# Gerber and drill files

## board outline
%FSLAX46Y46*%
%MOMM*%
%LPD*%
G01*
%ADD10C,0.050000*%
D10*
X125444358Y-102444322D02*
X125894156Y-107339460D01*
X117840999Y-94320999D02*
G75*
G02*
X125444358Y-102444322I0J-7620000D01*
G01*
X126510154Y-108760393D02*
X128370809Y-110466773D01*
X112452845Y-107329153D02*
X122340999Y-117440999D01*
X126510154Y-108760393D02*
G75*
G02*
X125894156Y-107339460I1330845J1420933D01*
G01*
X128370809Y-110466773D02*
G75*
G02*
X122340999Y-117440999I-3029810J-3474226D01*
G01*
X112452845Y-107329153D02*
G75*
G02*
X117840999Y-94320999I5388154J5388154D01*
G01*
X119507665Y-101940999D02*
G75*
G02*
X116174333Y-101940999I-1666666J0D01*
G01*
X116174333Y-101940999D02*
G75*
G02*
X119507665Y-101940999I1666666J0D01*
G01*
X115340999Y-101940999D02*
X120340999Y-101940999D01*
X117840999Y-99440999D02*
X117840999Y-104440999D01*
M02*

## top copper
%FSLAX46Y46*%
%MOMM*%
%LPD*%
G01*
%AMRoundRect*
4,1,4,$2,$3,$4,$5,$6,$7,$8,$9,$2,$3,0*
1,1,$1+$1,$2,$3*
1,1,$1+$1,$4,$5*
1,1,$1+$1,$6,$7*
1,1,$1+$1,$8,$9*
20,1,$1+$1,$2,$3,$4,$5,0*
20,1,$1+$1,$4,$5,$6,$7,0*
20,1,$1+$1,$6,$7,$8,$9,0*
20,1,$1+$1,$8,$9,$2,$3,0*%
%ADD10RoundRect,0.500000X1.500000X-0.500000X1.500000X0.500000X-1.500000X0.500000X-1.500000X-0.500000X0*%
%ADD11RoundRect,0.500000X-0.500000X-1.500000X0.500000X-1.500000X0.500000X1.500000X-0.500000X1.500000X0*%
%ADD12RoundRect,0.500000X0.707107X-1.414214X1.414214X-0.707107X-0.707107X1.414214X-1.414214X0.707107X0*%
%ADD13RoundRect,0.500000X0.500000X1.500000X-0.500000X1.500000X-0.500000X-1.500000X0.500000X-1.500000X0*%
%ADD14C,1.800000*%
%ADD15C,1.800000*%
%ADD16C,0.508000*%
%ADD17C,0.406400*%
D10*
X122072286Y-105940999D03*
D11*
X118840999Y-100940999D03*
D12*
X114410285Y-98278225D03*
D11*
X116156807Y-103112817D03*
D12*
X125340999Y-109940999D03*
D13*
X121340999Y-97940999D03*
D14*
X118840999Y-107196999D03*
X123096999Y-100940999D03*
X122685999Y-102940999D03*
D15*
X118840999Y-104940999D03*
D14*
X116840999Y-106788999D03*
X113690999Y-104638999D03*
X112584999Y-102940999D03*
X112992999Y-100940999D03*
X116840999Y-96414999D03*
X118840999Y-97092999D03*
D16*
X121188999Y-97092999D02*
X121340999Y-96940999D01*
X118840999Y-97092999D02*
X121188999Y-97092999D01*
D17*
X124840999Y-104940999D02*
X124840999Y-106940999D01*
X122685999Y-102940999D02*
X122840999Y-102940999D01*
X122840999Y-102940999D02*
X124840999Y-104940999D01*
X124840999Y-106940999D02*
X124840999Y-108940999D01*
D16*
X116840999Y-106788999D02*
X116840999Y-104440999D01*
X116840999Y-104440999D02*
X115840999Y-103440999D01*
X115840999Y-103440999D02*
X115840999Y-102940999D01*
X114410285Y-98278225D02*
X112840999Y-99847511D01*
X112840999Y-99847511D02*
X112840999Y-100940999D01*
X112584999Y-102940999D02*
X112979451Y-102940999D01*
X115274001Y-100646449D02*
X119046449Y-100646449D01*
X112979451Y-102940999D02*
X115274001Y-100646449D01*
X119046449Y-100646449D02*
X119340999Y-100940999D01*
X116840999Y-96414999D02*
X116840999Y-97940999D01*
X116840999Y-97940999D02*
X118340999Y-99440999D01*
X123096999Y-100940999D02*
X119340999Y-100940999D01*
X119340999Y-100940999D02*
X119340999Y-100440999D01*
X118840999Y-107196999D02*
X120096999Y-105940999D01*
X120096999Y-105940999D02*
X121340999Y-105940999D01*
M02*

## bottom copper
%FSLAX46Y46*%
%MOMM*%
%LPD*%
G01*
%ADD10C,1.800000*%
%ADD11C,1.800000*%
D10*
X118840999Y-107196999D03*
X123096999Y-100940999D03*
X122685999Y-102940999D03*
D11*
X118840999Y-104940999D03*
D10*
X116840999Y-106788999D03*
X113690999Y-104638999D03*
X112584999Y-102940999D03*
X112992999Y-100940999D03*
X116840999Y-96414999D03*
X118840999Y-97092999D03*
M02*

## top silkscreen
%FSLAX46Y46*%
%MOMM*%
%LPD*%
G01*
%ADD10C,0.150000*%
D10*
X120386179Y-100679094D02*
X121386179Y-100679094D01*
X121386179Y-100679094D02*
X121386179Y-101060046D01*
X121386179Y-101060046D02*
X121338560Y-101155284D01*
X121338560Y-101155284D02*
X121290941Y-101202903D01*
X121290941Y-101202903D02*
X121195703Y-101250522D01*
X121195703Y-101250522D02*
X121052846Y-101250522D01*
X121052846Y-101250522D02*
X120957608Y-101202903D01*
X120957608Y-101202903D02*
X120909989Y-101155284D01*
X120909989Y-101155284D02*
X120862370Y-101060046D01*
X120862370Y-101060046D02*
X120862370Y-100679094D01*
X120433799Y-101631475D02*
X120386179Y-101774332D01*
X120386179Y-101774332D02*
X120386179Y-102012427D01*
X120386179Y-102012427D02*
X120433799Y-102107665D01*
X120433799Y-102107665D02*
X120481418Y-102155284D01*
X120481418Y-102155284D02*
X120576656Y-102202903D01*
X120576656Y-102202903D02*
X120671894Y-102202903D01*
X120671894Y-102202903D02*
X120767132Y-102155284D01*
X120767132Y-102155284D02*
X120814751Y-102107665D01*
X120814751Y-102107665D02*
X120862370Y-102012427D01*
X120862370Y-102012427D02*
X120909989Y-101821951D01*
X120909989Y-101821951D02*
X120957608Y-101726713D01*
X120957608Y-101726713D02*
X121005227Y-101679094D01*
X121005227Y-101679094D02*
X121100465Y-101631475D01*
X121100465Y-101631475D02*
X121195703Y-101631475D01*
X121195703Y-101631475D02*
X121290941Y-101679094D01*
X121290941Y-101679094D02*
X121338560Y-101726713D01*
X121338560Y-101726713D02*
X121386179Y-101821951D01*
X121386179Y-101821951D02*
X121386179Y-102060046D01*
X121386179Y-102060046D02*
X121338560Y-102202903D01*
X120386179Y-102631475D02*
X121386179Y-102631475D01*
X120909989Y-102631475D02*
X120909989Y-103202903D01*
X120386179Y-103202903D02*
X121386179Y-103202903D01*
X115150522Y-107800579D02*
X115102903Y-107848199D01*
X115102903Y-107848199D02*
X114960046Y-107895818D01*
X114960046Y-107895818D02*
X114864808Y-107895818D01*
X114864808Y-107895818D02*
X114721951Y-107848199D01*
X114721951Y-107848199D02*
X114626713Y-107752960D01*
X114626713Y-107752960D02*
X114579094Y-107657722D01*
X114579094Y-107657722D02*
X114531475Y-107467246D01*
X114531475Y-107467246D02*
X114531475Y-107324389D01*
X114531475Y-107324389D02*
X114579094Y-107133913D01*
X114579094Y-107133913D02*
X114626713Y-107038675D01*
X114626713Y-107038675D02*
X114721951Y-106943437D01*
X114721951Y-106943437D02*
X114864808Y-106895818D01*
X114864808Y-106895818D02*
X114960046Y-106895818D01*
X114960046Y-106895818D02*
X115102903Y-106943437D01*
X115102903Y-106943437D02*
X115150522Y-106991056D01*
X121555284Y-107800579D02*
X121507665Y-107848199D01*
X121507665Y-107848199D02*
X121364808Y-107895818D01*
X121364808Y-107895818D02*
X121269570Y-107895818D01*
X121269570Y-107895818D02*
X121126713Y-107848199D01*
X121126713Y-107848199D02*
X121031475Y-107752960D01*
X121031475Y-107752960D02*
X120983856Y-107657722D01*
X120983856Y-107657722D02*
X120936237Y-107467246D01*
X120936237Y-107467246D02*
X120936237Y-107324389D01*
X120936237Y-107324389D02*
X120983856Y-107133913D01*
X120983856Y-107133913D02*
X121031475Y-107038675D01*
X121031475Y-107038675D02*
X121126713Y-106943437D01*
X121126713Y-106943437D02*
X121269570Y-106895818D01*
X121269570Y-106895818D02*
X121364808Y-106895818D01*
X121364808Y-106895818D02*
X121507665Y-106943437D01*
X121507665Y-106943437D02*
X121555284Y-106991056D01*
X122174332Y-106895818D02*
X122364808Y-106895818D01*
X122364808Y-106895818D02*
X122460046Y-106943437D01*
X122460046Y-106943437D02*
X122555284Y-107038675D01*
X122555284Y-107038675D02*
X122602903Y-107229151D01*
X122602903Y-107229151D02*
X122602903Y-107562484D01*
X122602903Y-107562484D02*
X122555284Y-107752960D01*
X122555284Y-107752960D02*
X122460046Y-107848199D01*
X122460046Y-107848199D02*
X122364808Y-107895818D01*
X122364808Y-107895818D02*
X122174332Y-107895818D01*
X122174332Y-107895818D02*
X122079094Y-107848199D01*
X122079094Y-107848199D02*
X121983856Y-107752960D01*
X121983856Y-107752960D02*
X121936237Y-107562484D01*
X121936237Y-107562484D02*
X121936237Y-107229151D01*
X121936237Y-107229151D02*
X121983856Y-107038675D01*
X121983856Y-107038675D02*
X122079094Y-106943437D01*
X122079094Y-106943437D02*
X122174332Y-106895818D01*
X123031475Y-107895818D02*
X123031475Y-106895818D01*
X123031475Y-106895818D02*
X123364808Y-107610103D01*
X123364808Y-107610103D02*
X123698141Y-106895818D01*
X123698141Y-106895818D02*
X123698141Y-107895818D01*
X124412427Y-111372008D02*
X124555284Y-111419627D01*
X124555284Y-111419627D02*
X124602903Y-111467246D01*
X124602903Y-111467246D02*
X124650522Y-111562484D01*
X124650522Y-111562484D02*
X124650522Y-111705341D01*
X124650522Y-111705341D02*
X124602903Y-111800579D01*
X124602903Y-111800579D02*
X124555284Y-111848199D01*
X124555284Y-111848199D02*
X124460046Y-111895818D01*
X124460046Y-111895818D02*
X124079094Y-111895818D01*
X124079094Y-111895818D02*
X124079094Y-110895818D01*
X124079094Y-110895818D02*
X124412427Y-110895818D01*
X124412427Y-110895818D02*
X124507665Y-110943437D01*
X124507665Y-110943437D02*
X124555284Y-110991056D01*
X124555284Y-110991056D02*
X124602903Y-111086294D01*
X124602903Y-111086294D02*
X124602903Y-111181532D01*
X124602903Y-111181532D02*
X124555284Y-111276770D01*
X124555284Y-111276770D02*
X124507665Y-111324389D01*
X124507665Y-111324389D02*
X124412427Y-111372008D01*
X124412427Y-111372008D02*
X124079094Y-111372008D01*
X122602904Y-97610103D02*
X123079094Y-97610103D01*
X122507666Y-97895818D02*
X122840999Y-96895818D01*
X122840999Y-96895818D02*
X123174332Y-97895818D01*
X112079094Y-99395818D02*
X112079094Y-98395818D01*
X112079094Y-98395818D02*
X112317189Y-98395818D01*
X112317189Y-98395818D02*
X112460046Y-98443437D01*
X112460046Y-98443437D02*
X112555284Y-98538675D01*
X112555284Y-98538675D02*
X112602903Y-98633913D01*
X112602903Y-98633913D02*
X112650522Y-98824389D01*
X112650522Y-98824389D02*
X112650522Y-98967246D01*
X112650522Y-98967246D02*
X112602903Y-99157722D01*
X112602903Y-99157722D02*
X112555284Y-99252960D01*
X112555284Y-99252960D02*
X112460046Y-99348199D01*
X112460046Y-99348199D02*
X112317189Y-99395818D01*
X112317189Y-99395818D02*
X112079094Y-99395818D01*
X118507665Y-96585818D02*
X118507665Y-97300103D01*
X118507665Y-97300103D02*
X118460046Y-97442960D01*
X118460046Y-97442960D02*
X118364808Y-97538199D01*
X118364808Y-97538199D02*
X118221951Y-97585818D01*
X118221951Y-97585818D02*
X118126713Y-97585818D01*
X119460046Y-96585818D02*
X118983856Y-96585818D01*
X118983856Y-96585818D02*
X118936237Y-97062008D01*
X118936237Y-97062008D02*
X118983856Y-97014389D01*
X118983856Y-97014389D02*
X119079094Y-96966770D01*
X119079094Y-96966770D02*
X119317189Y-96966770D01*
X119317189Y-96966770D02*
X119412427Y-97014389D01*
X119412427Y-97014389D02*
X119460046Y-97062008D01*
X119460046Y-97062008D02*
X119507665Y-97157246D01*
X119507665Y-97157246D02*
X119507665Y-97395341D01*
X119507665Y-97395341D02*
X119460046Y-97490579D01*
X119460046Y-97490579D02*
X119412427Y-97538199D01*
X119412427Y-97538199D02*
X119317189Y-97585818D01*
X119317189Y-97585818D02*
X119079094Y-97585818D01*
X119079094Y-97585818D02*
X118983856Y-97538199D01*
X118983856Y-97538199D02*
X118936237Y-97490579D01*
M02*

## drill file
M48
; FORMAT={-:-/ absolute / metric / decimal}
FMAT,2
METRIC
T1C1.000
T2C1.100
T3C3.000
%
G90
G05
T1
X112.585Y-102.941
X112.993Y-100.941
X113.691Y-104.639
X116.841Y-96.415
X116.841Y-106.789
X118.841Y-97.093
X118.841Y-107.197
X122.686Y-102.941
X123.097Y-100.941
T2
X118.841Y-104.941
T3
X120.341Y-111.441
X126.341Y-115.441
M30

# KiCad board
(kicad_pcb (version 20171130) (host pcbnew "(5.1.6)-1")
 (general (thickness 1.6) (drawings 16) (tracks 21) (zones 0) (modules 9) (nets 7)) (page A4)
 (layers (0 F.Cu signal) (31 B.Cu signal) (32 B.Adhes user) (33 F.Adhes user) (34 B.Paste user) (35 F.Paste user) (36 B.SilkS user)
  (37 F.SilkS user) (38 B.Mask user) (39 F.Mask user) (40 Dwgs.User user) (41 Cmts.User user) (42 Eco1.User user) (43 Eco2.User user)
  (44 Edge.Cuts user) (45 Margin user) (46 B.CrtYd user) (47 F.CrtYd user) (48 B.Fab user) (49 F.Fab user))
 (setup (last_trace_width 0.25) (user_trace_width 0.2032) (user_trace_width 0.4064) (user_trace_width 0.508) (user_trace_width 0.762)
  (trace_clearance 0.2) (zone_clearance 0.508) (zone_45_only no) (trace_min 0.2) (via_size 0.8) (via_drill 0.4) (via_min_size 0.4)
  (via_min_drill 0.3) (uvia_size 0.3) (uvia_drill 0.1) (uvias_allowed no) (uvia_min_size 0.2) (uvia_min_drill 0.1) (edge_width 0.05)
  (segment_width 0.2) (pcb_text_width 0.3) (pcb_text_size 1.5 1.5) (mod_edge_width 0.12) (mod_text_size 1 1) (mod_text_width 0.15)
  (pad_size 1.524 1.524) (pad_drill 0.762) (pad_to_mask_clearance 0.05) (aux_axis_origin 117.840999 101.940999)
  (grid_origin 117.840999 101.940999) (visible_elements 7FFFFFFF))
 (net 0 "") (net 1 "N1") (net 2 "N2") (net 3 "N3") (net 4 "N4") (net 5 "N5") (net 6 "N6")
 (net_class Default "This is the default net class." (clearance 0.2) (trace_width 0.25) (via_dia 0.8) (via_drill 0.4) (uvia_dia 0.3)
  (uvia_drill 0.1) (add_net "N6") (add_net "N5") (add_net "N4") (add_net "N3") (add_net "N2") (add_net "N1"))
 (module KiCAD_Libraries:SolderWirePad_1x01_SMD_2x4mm (layer F.Cu) (at 122.072286 105.940999 90)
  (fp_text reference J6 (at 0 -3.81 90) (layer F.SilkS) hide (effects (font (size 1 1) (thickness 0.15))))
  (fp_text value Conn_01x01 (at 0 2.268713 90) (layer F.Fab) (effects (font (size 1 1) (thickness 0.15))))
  (pad 1 smd roundrect (at 0 0 90) (size 2 4) (layers F.Cu F.Paste F.Mask) (roundrect_rratio 0.25) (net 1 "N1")))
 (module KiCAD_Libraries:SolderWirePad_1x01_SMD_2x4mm (layer F.Cu) (at 118.840999 100.940999)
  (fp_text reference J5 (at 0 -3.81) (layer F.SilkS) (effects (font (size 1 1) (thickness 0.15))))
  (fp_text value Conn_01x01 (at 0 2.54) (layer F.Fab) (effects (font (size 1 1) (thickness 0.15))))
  (pad 1 smd roundrect (at 0 0) (size 2 4) (layers F.Cu F.Paste F.Mask) (roundrect_rratio 0.25) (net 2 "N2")))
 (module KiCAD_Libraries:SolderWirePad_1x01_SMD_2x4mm (layer F.Cu) (at 114.410285 98.278225 45)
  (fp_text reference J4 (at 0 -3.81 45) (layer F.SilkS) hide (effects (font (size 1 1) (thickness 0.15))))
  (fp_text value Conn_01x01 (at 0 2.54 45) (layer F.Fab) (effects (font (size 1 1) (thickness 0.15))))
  (pad 1 smd roundrect (at 0 0 45) (size 2 4) (layers F.Cu F.Paste F.Mask) (roundrect_rratio 0.25) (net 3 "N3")))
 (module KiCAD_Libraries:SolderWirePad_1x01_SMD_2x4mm (layer F.Cu) (at 116.156807 103.112817)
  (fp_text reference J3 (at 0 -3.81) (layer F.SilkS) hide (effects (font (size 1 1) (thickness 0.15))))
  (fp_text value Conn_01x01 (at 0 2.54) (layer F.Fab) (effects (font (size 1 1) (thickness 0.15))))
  (pad 1 smd roundrect (at 0 0) (size 2 4) (layers F.Cu F.Paste F.Mask) (roundrect_rratio 0.25) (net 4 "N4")))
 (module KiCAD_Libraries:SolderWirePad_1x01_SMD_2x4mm (layer F.Cu) (at 125.340999 109.940999 45)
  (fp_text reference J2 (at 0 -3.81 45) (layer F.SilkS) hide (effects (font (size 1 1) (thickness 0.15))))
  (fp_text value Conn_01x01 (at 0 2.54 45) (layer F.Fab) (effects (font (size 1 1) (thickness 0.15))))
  (pad 1 smd roundrect (at 0 0 45) (size 2 4) (layers F.Cu F.Paste F.Mask) (roundrect_rratio 0.25) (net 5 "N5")))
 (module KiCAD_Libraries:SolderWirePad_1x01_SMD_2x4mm (layer F.Cu) (at 121.340999 97.940999 180)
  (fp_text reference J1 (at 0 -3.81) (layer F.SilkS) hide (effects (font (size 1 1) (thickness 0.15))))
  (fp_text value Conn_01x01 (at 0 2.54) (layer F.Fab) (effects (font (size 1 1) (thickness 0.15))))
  (pad 1 smd roundrect (at 0 0 180) (size 2 4) (layers F.Cu F.Paste F.Mask) (roundrect_rratio 0.25) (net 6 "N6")))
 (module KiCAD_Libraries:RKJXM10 (layer B.Cu) (at 117.840999 101.940999)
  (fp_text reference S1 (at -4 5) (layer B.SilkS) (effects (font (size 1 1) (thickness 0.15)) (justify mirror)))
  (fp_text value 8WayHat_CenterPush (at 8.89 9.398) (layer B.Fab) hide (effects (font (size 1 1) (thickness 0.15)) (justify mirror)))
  (pad COM thru_hole circle (at 1 5.256) (size 1.8 1.8) (drill 1) (layers *.Cu *.Mask) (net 1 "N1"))
  (pad PUSH3 thru_hole circle (at 5.256 -1) (size 1.8 1.8) (drill 1) (layers *.Cu *.Mask) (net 2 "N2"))
  (pad B thru_hole circle (at 4.845 1) (size 1.8 1.8) (drill 1) (layers *.Cu *.Mask) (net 5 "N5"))
  (pad "" np_thru_hole circle (at 1 3) (size 1.8 1.8) (drill 1.1) (layers *.Cu *.Mask))
  (pad C thru_hole circle (at -1 4.848) (size 1.8 1.8) (drill 1) (layers *.Cu *.Mask) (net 4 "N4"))
  (pad GND thru_hole circle (at -4.15 2.698) (size 1.8 1.8) (drill 1) (layers *.Cu *.Mask))
  (pad PUSH1 thru_hole circle (at -5.256 1) (size 1.8 1.8) (drill 1) (layers *.Cu *.Mask) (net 2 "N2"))
  (pad D thru_hole circle (at -4.848 -1) (size 1.8 1.8) (drill 1) (layers *.Cu *.Mask) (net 3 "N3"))
  (pad PUSH2 thru_hole circle (at -1 -5.526) (size 1.8 1.8) (drill 1) (layers *.Cu *.Mask) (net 2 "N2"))
  (pad A thru_hole circle (at 1 -4.848) (size 1.8 1.8) (drill 1) (layers *.Cu *.Mask) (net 6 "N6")))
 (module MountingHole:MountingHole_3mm (layer B.Cu) (at 120.340999 111.440999)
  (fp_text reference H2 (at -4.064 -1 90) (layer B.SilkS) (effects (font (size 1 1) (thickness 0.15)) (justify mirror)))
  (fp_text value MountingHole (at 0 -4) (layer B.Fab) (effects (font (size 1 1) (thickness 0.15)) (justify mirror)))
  (pad 1 np_thru_hole circle (at 0 0) (size 3 3) (drill 3) (layers *.Cu *.Mask)))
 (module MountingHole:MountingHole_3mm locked (layer B.Cu) (at 126.340999 115.440999)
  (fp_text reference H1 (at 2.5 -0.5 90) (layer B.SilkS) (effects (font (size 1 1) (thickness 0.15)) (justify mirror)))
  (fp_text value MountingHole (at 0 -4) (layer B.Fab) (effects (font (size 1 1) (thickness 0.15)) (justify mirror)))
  (pad 1 np_thru_hole circle (at 0 0) (size 3 3) (drill 3) (layers *.Cu *.Mask)))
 (gr_line (start 125.444358 102.444322) (end 125.894156 107.33946) (layer Edge.Cuts) (width 0.05))
 (gr_arc (start 117.840999 101.940999) (end 117.840999 94.320999) (angle 93.78731084) (layer Edge.Cuts) (width 0.05))
 (gr_line (start 126.510154 108.760393) (end 128.370809 110.466773) (layer Edge.Cuts) (width 0.05))
 (gr_line (start 112.452845 107.329153) (end 122.340999 117.440999) (layer Edge.Cuts) (width 0.05))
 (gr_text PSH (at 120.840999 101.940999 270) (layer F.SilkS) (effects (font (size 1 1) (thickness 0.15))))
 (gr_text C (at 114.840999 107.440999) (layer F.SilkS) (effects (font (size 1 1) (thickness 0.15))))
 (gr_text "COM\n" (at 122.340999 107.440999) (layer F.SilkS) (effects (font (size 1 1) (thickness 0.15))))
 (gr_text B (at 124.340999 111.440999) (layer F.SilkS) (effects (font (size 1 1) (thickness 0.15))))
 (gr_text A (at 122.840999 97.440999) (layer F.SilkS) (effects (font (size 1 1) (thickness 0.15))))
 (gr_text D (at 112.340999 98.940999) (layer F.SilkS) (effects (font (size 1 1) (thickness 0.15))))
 (gr_arc (start 127.840999 107.33946) (end 125.894156 107.33946) (angle -46.87509459) (layer Edge.Cuts) (width 0.05))
 (gr_arc (start 125.340999 113.940999) (end 122.340999 117.440999) (angle -179.5101973) (layer Edge.Cuts) (width 0.05))
 (gr_arc (start 117.840999 101.940999) (end 117.840999 94.320999) (angle -135) (layer Edge.Cuts) (width 0.05))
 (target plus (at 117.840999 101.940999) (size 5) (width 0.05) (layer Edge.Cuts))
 (segment (start 121.188999 97.092999) (end 121.340999 96.940999) (width 0.508) (layer F.Cu) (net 6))
 (segment (start 118.840999 97.092999) (end 121.188999 97.092999) (width 0.508) (layer F.Cu) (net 6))
 (segment (start 124.840999 104.940999) (end 124.840999 106.940999) (width 0.4064) (layer F.Cu) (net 5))
 (segment (start 122.685999 102.940999) (end 122.840999 102.940999) (width 0.4064) (layer F.Cu) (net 5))
 (segment (start 122.840999 102.940999) (end 124.840999 104.940999) (width 0.4064) (layer F.Cu) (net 5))
 (segment (start 124.840999 106.940999) (end 124.840999 108.940999) (width 0.4064) (layer F.Cu) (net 5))
 (segment (start 116.840999 106.788999) (end 116.840999 104.440999) (width 0.508) (layer F.Cu) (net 4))
 (segment (start 116.840999 104.440999) (end 115.840999 103.440999) (width 0.508) (layer F.Cu) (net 4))
 (segment (start 115.840999 103.440999) (end 115.840999 102.940999) (width 0.508) (layer F.Cu) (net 4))
 (segment (start 114.410285 98.278225) (end 112.840999 99.847511) (width 0.508) (layer F.Cu) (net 3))
 (segment (start 112.840999 99.847511) (end 112.840999 100.940999) (width 0.508) (layer F.Cu) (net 3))
 (segment (start 112.584999 102.940999) (end 112.979451 102.940999) (width 0.508) (layer F.Cu) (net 2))
 (segment (start 115.274001 100.646449) (end 119.046449 100.646449) (width 0.508) (layer F.Cu) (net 2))
 (segment (start 112.979451 102.940999) (end 115.274001 100.646449) (width 0.508) (layer F.Cu) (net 2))
 (segment (start 119.046449 100.646449) (end 119.340999 100.940999) (width 0.508) (layer F.Cu) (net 2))
 (segment (start 116.840999 96.414999) (end 116.840999 97.940999) (width 0.508) (layer F.Cu) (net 2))
 (segment (start 116.840999 97.940999) (end 118.340999 99.440999) (width 0.508) (layer F.Cu) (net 2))
 (segment (start 123.096999 100.940999) (end 119.340999 100.940999) (width 0.508) (layer F.Cu) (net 2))
 (segment (start 119.340999 100.940999) (end 119.340999 100.440999) (width 0.508) (layer F.Cu) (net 2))
 (segment (start 118.840999 107.196999) (end 120.096999 105.940999) (width 0.508) (layer F.Cu) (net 1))
 (segment (start 120.096999 105.940999) (end 121.340999 105.940999) (width 0.508) (layer F.Cu) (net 1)))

